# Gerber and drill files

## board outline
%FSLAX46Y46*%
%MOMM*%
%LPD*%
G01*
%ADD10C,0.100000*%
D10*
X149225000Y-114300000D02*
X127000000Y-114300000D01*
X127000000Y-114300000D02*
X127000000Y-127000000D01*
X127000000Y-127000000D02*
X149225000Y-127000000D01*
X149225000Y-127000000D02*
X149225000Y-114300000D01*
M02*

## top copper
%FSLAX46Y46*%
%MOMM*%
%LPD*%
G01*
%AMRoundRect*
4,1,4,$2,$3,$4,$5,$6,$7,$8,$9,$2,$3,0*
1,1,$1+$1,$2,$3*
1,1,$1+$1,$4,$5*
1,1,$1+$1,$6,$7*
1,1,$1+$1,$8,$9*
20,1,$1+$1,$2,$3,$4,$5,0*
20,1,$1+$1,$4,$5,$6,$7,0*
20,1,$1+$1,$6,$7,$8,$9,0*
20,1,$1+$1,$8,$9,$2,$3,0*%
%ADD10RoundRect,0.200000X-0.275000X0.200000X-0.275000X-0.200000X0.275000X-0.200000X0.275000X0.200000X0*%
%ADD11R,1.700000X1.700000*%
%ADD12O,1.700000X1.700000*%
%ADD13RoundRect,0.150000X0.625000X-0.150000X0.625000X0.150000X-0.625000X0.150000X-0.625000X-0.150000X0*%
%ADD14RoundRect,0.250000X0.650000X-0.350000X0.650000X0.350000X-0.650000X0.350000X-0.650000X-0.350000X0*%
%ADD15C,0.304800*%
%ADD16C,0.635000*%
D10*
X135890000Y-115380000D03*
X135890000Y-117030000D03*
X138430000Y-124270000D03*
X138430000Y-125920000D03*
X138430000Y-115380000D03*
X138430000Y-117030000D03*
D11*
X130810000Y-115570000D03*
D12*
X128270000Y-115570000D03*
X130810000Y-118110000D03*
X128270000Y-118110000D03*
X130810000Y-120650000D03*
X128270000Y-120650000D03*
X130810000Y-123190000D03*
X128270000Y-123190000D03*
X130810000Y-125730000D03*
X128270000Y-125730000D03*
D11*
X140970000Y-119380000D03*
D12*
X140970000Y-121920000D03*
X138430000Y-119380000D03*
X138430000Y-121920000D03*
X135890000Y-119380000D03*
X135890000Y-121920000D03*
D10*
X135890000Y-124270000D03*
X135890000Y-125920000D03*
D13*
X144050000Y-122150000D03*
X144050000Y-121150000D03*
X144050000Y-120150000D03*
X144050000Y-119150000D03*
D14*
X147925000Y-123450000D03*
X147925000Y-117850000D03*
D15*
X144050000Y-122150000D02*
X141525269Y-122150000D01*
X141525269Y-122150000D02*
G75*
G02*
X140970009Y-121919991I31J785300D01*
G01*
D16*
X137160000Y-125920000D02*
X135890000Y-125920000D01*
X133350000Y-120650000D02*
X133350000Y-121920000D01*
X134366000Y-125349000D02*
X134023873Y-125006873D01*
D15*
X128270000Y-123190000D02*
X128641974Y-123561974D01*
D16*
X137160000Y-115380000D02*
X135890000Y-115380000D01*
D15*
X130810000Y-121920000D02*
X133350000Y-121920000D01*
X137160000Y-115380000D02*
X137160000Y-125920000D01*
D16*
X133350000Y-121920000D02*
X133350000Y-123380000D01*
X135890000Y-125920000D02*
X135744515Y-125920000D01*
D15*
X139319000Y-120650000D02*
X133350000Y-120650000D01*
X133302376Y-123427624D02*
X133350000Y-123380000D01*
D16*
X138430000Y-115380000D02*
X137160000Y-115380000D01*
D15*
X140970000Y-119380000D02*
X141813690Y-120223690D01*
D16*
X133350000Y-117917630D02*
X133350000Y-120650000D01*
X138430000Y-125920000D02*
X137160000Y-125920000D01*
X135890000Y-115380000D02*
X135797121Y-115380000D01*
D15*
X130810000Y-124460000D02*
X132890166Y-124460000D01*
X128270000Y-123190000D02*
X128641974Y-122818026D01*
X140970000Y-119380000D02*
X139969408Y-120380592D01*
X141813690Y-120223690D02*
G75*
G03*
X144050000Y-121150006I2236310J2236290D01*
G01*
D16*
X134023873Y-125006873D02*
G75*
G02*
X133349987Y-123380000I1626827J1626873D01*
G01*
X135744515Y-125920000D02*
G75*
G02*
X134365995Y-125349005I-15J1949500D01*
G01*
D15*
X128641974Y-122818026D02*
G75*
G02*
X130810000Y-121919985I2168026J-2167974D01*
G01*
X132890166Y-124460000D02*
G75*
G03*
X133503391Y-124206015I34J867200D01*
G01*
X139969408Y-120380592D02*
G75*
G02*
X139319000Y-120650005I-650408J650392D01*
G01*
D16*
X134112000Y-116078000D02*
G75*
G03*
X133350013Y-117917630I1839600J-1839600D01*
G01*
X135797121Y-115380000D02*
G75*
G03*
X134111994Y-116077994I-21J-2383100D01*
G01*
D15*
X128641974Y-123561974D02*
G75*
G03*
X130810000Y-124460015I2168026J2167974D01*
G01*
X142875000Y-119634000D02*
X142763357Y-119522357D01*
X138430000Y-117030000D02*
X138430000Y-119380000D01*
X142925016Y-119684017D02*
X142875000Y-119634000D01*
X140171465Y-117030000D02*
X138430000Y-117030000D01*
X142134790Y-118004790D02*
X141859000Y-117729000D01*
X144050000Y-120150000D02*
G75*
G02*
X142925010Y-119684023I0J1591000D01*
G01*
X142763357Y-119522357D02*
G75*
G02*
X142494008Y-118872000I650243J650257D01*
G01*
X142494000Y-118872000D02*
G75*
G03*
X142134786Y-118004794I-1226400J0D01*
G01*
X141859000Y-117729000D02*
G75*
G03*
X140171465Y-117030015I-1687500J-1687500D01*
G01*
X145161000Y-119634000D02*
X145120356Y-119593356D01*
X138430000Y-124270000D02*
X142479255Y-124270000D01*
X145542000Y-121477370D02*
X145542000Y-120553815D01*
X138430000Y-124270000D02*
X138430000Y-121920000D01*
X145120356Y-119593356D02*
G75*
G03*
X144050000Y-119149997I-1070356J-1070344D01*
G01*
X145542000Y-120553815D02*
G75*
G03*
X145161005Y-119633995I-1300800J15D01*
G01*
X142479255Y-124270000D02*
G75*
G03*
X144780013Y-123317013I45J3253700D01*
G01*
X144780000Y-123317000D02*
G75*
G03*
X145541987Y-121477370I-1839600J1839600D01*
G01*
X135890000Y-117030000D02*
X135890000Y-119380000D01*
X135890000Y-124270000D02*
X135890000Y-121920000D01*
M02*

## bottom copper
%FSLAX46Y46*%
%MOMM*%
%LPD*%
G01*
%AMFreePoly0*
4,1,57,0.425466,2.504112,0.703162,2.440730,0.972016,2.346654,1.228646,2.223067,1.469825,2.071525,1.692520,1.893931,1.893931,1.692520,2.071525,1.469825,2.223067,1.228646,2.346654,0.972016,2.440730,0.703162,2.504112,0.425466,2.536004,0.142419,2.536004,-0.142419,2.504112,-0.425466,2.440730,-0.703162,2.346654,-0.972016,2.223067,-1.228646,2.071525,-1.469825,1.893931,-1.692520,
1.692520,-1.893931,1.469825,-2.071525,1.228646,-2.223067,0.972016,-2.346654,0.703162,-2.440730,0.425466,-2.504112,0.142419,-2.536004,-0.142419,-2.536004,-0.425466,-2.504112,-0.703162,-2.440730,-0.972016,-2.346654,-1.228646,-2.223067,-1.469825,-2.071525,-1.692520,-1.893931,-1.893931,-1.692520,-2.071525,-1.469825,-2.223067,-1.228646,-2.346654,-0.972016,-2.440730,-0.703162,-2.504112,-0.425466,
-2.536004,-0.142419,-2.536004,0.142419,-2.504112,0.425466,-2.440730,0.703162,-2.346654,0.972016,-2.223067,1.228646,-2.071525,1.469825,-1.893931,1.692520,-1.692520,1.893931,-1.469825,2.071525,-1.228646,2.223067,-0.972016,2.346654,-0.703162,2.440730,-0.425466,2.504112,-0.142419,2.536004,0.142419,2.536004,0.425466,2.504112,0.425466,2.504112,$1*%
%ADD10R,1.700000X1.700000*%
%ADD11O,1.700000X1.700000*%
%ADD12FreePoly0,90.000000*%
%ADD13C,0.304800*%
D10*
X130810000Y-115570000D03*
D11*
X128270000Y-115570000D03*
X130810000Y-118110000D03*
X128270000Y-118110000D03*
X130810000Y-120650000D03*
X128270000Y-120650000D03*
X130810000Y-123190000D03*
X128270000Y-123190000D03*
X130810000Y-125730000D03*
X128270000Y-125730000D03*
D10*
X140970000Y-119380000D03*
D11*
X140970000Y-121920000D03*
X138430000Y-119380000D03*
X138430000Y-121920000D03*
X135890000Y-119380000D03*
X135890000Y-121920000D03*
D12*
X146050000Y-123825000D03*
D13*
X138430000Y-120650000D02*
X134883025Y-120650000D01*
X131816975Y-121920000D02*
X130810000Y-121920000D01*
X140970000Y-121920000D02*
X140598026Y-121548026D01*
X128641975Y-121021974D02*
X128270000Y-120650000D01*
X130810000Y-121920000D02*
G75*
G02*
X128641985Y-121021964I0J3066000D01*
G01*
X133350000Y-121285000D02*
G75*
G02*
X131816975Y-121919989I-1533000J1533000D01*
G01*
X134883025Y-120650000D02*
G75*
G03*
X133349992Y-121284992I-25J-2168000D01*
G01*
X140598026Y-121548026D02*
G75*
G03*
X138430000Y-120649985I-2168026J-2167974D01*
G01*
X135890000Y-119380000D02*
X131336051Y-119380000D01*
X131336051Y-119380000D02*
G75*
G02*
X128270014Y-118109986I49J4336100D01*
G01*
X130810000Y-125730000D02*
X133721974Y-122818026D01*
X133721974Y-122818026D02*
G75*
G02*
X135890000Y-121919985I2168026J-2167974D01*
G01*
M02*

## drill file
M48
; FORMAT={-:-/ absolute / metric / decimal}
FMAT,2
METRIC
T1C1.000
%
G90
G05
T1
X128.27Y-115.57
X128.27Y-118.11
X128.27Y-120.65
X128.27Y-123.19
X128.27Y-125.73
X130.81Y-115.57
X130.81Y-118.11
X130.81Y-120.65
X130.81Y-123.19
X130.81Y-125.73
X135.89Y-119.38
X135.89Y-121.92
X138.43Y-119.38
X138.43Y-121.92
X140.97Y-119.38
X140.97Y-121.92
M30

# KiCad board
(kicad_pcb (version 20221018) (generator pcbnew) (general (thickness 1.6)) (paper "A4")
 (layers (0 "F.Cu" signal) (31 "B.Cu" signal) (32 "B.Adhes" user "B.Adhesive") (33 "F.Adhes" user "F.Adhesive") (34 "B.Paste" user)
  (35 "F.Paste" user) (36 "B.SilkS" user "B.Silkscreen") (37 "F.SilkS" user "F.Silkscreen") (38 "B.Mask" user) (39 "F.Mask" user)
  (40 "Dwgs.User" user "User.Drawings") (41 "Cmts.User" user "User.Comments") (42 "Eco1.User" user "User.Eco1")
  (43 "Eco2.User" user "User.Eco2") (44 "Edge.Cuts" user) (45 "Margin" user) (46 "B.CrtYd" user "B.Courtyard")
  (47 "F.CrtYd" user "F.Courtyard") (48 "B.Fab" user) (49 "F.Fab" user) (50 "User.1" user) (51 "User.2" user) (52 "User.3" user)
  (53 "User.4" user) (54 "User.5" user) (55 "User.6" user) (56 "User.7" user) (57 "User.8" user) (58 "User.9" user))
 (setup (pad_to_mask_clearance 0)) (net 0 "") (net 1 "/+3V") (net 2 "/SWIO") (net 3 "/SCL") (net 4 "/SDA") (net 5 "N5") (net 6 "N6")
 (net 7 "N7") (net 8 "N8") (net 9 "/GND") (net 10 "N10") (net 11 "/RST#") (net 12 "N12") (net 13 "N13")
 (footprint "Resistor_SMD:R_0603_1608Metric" (layer "F.Cu") (at 135.89 116.205 -90)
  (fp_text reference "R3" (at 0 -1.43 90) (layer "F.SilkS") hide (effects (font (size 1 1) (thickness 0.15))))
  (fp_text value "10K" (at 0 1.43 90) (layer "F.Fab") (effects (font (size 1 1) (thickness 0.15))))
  (pad "1" smd roundrect (at -0.825 0 270) (size 0.8 0.95) (layers "F.Cu" "F.Paste" "F.Mask") (roundrect_rratio 0.25) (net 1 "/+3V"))
  (pad "2" smd roundrect (at 0.825 0 270) (size 0.8 0.95) (layers "F.Cu" "F.Paste" "F.Mask") (roundrect_rratio 0.25) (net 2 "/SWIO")))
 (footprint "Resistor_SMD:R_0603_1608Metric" (layer "F.Cu") (at 138.43 125.095 -90)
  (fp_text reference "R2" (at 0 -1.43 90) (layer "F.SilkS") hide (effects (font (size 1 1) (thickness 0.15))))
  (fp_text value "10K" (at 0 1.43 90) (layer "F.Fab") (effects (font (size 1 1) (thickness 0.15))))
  (pad "1" smd roundrect (at -0.825 0 270) (size 0.8 0.95) (layers "F.Cu" "F.Paste" "F.Mask") (roundrect_rratio 0.25) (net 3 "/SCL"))
  (pad "2" smd roundrect (at 0.825 0 270) (size 0.8 0.95) (layers "F.Cu" "F.Paste" "F.Mask") (roundrect_rratio 0.25) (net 1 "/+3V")))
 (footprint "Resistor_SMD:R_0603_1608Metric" (layer "F.Cu") (at 138.43 116.205 -90)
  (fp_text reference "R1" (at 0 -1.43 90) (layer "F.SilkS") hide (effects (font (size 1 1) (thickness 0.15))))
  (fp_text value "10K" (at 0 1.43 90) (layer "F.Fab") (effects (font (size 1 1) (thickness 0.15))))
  (pad "1" smd roundrect (at -0.825 0 270) (size 0.8 0.95) (layers "F.Cu" "F.Paste" "F.Mask") (roundrect_rratio 0.25) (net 1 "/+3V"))
  (pad "2" smd roundrect (at 0.825 0 270) (size 0.8 0.95) (layers "F.Cu" "F.Paste" "F.Mask") (roundrect_rratio 0.25) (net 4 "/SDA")))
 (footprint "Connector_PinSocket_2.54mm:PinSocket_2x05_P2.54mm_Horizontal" (layer "F.Cu") (at 130.81 115.57)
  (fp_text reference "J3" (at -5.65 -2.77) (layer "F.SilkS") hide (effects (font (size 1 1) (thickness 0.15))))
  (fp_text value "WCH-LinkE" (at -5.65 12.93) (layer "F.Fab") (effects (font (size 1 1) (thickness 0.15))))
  (pad "1" thru_hole rect (at 0 0) (size 1.7 1.7) (drill 1) (layers "*.Cu" "*.Mask") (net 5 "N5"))
  (pad "2" thru_hole oval (at -2.54 0) (size 1.7 1.7) (drill 1) (layers "*.Cu" "*.Mask") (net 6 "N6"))
  (pad "3" thru_hole oval (at 0 2.54) (size 1.7 1.7) (drill 1) (layers "*.Cu" "*.Mask") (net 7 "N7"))
  (pad "4" thru_hole oval (at -2.54 2.54) (size 1.7 1.7) (drill 1) (layers "*.Cu" "*.Mask") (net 2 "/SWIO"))
  (pad "5" thru_hole oval (at 0 5.08) (size 1.7 1.7) (drill 1) (layers "*.Cu" "*.Mask") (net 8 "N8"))
  (pad "6" thru_hole oval (at -2.54 5.08) (size 1.7 1.7) (drill 1) (layers "*.Cu" "*.Mask") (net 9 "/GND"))
  (pad "7" thru_hole oval (at 0 7.62) (size 1.7 1.7) (drill 1) (layers "*.Cu" "*.Mask") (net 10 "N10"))
  (pad "8" thru_hole oval (at -2.54 7.62) (size 1.7 1.7) (drill 1) (layers "*.Cu" "*.Mask") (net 1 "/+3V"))
  (pad "9" thru_hole oval (at 0 10.16) (size 1.7 1.7) (drill 1) (layers "*.Cu" "*.Mask") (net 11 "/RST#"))
  (pad "10" thru_hole oval (at -2.54 10.16) (size 1.7 1.7) (drill 1) (layers "*.Cu" "*.Mask") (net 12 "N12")))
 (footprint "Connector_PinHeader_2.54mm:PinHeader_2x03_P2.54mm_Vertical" (layer "F.Cu") (at 140.97 119.38 -90)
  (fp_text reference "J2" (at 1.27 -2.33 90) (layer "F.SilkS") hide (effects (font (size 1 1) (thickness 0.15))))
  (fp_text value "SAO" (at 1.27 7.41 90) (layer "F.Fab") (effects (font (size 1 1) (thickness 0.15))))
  (pad "1" thru_hole rect (at 0 0 270) (size 1.7 1.7) (drill 1) (layers "*.Cu" "*.Mask") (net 1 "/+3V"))
  (pad "2" thru_hole oval (at 2.54 0 270) (size 1.7 1.7) (drill 1) (layers "*.Cu" "*.Mask") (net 9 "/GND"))
  (pad "3" thru_hole oval (at 0 2.54 270) (size 1.7 1.7) (drill 1) (layers "*.Cu" "*.Mask") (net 4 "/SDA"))
  (pad "4" thru_hole oval (at 2.54 2.54 270) (size 1.7 1.7) (drill 1) (layers "*.Cu" "*.Mask") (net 3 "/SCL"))
  (pad "5" thru_hole oval (at 0 5.08 270) (size 1.7 1.7) (drill 1) (layers "*.Cu" "*.Mask") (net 2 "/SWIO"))
  (pad "6" thru_hole oval (at 2.54 5.08 270) (size 1.7 1.7) (drill 1) (layers "*.Cu" "*.Mask") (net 11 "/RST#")))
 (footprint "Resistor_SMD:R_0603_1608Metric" (layer "F.Cu") (at 135.89 125.095 -90)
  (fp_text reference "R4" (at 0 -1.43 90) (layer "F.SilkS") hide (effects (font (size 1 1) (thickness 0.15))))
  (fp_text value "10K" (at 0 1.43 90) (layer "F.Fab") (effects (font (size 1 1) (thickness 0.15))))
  (pad "1" smd roundrect (at -0.825 0 270) (size 0.8 0.95) (layers "F.Cu" "F.Paste" "F.Mask") (roundrect_rratio 0.25) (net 11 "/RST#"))
  (pad "2" smd roundrect (at 0.825 0 270) (size 0.8 0.95) (layers "F.Cu" "F.Paste" "F.Mask") (roundrect_rratio 0.25) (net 1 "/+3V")))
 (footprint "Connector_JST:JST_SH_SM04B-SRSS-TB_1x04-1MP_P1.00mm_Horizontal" (layer "F.Cu") (at 146.05 120.65 90)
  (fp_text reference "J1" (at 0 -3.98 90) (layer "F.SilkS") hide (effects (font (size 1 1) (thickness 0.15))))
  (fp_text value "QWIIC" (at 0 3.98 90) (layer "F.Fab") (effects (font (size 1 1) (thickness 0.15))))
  (pad "1" smd roundrect (at -1.5 -2 90) (size 0.6 1.55) (layers "F.Cu" "F.Paste" "F.Mask") (roundrect_rratio 0.25) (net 9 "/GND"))
  (pad "2" smd roundrect (at -0.5 -2 90) (size 0.6 1.55) (layers "F.Cu" "F.Paste" "F.Mask") (roundrect_rratio 0.25) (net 1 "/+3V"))
  (pad "3" smd roundrect (at 0.5 -2 90) (size 0.6 1.55) (layers "F.Cu" "F.Paste" "F.Mask") (roundrect_rratio 0.25) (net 4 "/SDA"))
  (pad "4" smd roundrect (at 1.5 -2 90) (size 0.6 1.55) (layers "F.Cu" "F.Paste" "F.Mask") (roundrect_rratio 0.25) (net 3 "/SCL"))
  (pad "MP" smd roundrect (at -2.8 1.875 90) (size 1.2 1.8) (layers "F.Cu" "F.Paste" "F.Mask") (roundrect_rratio 0.208333))
  (pad "MP" smd roundrect (at 2.8 1.875 90) (size 1.2 1.8) (layers "F.Cu" "F.Paste" "F.Mask") (roundrect_rratio 0.208333)))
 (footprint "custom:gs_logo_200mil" (layer "B.Cu") (at 146.05 123.825 90)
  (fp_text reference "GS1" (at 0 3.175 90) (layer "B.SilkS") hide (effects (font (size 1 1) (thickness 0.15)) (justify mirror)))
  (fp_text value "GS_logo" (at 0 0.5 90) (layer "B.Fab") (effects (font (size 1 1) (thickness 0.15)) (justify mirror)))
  (pad "1" smd custom (at 0 0 90) (size 5.08 5.08) (layers "B.Cu") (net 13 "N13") (zone_connect 0) (thermal_bridge_angle 45)
   (options (clearance outline) (anchor circle)) (primitives)))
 (gr_line (start 149.225 114.3) (end 127 114.3) (stroke (width 0.1) (type default)) (layer "Edge.Cuts"))
 (gr_line (start 127 114.3) (end 127 127) (stroke (width 0.1) (type default)) (layer "Edge.Cuts"))
 (gr_line (start 127 127) (end 149.225 127) (stroke (width 0.1) (type default)) (layer "Edge.Cuts"))
 (gr_line (start 149.225 127) (end 149.225 114.3) (stroke (width 0.1) (type default)) (layer "Edge.Cuts"))
 (segment (start 144.05 122.15) (end 141.525269 122.15) (width 0.3048) (layer "F.Cu") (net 9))
 (arc (start 141.525269 122.15) (mid 141.22476 122.090225) (end 140.97 121.92) (width 0.3048) (layer "F.Cu") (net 9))
 (segment (start 138.43 120.65) (end 134.883025 120.65) (width 0.3048) (layer "B.Cu") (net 9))
 (segment (start 131.816975 121.92) (end 130.81 121.92) (width 0.3048) (layer "B.Cu") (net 9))
 (segment (start 140.97 121.92) (end 140.598026 121.548026) (width 0.3048) (layer "B.Cu") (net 9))
 (segment (start 128.641975 121.021974) (end 128.27 120.65) (width 0.3048) (layer "B.Cu") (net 9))
 (arc (start 130.81 121.92) (mid 129.636673 121.686611) (end 128.641975 121.021974) (width 0.3048) (layer "B.Cu") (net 9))
 (arc (start 133.35 121.285) (mid 132.646643 121.754968) (end 131.816975 121.92) (width 0.3048) (layer "B.Cu") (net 9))
 (arc (start 134.883025 120.65) (mid 134.053358 120.815031) (end 133.35 121.285) (width 0.3048) (layer "B.Cu") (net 9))
 (arc (start 140.598026 121.548026) (mid 139.603328 120.883389) (end 138.43 120.65) (width 0.3048) (layer "B.Cu") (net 9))
 (segment (start 137.16 125.92) (end 135.89 125.92) (width 0.635) (layer "F.Cu") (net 1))
 (segment (start 133.35 120.65) (end 133.35 121.92) (width 0.635) (layer "F.Cu") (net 1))
 (segment (start 134.366 125.349) (end 134.023873 125.006873) (width 0.635) (layer "F.Cu") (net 1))
 (segment (start 128.27 123.19) (end 128.641974 123.561974) (width 0.3048) (layer "F.Cu") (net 1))
 (segment (start 137.16 115.38) (end 135.89 115.38) (width 0.635) (layer "F.Cu") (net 1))
 (segment (start 130.81 121.92) (end 133.35 121.92) (width 0.3048) (layer "F.Cu") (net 1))
 (segment (start 137.16 115.38) (end 137.16 125.92) (width 0.3048) (layer "F.Cu") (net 1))
 (segment (start 133.35 121.92) (end 133.35 123.38) (width 0.635) (layer "F.Cu") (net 1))
 (segment (start 135.89 125.92) (end 135.744515 125.92) (width 0.635) (layer "F.Cu") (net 1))
 (segment (start 139.319 120.65) (end 133.35 120.65) (width 0.3048) (layer "F.Cu") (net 1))
 (segment (start 133.302376 123.427624) (end 133.35 123.38) (width 0.3048) (layer "F.Cu") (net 1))
 (segment (start 138.43 115.38) (end 137.16 115.38) (width 0.635) (layer "F.Cu") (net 1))
 (segment (start 140.97 119.38) (end 141.81369 120.22369) (width 0.3048) (layer "F.Cu") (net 1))
 (segment (start 133.35 117.91763) (end 133.35 120.65) (width 0.635) (layer "F.Cu") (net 1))
 (segment (start 138.43 125.92) (end 137.16 125.92) (width 0.635) (layer "F.Cu") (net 1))
 (segment (start 135.89 115.38) (end 135.797121 115.38) (width 0.635) (layer "F.Cu") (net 1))
 (segment (start 130.81 124.46) (end 132.890166 124.46) (width 0.3048) (layer "F.Cu") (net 1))
 (segment (start 128.27 123.19) (end 128.641974 122.818026) (width 0.3048) (layer "F.Cu") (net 1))
 (segment (start 140.97 119.38) (end 139.969408 120.380592) (width 0.3048) (layer "F.Cu") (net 1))
 (arc (start 141.81369 120.22369) (mid 142.839717 120.90926) (end 144.05 121.15) (width 0.3048) (layer "F.Cu") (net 1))
 (arc (start 134.023873 125.006873) (mid 133.525134 124.260458) (end 133.35 123.38) (width 0.635) (layer "F.Cu") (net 1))
 (arc (start 135.744515 125.92) (mid 134.998468 125.771602) (end 134.366 125.349) (width 0.635) (layer "F.Cu") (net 1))
 (arc (start 128.641974 122.818026) (mid 129.636672 122.153389) (end 130.81 121.92) (width 0.3048) (layer "F.Cu") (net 1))
 (arc (start 132.890166 124.46) (mid 133.222033 124.393988) (end 133.503376 124.206) (width 0.3048) (layer "F.Cu") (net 1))
 (arc (start 139.969408 120.380592) (mid 139.670999 120.579983) (end 139.319 120.65) (width 0.3048) (layer "F.Cu") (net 1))
 (arc (start 134.112 116.078) (mid 133.548037 116.922029) (end 133.35 117.91763) (width 0.635) (layer "F.Cu") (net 1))
 (arc (start 135.797121 115.38) (mid 134.885141 115.561404) (end 134.112 116.078) (width 0.635) (layer "F.Cu") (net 1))
 (arc (start 128.641974 123.561974) (mid 129.636672 124.226611) (end 130.81 124.46) (width 0.3048) (layer "F.Cu") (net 1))
 (segment (start 142.875 119.634) (end 142.763357 119.522357) (width 0.3048) (layer "F.Cu") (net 4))
 (segment (start 138.43 117.03) (end 138.43 119.38) (width 0.3048) (layer "F.Cu") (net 4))
 (segment (start 142.925016 119.684017) (end 142.875 119.634) (width 0.3048) (layer "F.Cu") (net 4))
 (segment (start 140.171465 117.03) (end 138.43 117.03) (width 0.3048) (layer "F.Cu") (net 4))
 (segment (start 142.13479 118.00479) (end 141.859 117.729) (width 0.3048) (layer "F.Cu") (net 4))
 (arc (start 144.05 120.15) (mid 143.441163 120.028895) (end 142.925016 119.684017) (width 0.3048) (layer "F.Cu") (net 4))
 (arc (start 142.763357 119.522357) (mid 142.564003 119.224002) (end 142.494 118.872) (width 0.3048) (layer "F.Cu") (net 4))
 (arc (start 142.494 118.872) (mid 142.400644 118.402669) (end 142.13479 118.00479) (width 0.3048) (layer "F.Cu") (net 4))
 (arc (start 141.859 117.729) (mid 141.084753 117.211664) (end 140.171465 117.03) (width 0.3048) (layer "F.Cu") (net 4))
 (segment (start 145.161 119.634) (end 145.120356 119.593356) (width 0.3048) (layer "F.Cu") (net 3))
 (segment (start 138.43 124.27) (end 142.479255 124.27) (width 0.3048) (layer "F.Cu") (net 3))
 (segment (start 145.542 121.47737) (end 145.542 120.553815) (width 0.3048) (layer "F.Cu") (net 3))
 (segment (start 138.43 124.27) (end 138.43 121.92) (width 0.3048) (layer "F.Cu") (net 3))
 (arc (start 145.120356 119.593356) (mid 144.629273 119.265225) (end 144.05 119.15) (width 0.3048) (layer "F.Cu") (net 3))
 (arc (start 145.542 120.553815) (mid 145.442982 120.056015) (end 145.161 119.634) (width 0.3048) (layer "F.Cu") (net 3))
 (arc (start 142.479255 124.27) (mid 143.724409 124.022324) (end 144.78 123.317) (width 0.3048) (layer "F.Cu") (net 3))
 (arc (start 144.78 123.317) (mid 145.343963 122.472971) (end 145.542 121.47737) (width 0.3048) (layer "F.Cu") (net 3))
 (segment (start 135.89 117.03) (end 135.89 119.38) (width 0.3048) (layer "F.Cu") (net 2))
 (segment (start 135.89 119.38) (end 131.336051 119.38) (width 0.3048) (layer "B.Cu") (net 2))
 (arc (start 131.336051 119.38) (mid 129.676717 119.049938) (end 128.27 118.11) (width 0.3048) (layer "B.Cu") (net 2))
 (segment (start 135.89 124.27) (end 135.89 121.92) (width 0.3048) (layer "F.Cu") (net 11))
 (segment (start 130.81 125.73) (end 133.721974 122.818026) (width 0.3048) (layer "B.Cu") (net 11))
 (arc (start 133.721974 122.818026) (mid 134.716672 122.153389) (end 135.89 121.92) (width 0.3048) (layer "B.Cu") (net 11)))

